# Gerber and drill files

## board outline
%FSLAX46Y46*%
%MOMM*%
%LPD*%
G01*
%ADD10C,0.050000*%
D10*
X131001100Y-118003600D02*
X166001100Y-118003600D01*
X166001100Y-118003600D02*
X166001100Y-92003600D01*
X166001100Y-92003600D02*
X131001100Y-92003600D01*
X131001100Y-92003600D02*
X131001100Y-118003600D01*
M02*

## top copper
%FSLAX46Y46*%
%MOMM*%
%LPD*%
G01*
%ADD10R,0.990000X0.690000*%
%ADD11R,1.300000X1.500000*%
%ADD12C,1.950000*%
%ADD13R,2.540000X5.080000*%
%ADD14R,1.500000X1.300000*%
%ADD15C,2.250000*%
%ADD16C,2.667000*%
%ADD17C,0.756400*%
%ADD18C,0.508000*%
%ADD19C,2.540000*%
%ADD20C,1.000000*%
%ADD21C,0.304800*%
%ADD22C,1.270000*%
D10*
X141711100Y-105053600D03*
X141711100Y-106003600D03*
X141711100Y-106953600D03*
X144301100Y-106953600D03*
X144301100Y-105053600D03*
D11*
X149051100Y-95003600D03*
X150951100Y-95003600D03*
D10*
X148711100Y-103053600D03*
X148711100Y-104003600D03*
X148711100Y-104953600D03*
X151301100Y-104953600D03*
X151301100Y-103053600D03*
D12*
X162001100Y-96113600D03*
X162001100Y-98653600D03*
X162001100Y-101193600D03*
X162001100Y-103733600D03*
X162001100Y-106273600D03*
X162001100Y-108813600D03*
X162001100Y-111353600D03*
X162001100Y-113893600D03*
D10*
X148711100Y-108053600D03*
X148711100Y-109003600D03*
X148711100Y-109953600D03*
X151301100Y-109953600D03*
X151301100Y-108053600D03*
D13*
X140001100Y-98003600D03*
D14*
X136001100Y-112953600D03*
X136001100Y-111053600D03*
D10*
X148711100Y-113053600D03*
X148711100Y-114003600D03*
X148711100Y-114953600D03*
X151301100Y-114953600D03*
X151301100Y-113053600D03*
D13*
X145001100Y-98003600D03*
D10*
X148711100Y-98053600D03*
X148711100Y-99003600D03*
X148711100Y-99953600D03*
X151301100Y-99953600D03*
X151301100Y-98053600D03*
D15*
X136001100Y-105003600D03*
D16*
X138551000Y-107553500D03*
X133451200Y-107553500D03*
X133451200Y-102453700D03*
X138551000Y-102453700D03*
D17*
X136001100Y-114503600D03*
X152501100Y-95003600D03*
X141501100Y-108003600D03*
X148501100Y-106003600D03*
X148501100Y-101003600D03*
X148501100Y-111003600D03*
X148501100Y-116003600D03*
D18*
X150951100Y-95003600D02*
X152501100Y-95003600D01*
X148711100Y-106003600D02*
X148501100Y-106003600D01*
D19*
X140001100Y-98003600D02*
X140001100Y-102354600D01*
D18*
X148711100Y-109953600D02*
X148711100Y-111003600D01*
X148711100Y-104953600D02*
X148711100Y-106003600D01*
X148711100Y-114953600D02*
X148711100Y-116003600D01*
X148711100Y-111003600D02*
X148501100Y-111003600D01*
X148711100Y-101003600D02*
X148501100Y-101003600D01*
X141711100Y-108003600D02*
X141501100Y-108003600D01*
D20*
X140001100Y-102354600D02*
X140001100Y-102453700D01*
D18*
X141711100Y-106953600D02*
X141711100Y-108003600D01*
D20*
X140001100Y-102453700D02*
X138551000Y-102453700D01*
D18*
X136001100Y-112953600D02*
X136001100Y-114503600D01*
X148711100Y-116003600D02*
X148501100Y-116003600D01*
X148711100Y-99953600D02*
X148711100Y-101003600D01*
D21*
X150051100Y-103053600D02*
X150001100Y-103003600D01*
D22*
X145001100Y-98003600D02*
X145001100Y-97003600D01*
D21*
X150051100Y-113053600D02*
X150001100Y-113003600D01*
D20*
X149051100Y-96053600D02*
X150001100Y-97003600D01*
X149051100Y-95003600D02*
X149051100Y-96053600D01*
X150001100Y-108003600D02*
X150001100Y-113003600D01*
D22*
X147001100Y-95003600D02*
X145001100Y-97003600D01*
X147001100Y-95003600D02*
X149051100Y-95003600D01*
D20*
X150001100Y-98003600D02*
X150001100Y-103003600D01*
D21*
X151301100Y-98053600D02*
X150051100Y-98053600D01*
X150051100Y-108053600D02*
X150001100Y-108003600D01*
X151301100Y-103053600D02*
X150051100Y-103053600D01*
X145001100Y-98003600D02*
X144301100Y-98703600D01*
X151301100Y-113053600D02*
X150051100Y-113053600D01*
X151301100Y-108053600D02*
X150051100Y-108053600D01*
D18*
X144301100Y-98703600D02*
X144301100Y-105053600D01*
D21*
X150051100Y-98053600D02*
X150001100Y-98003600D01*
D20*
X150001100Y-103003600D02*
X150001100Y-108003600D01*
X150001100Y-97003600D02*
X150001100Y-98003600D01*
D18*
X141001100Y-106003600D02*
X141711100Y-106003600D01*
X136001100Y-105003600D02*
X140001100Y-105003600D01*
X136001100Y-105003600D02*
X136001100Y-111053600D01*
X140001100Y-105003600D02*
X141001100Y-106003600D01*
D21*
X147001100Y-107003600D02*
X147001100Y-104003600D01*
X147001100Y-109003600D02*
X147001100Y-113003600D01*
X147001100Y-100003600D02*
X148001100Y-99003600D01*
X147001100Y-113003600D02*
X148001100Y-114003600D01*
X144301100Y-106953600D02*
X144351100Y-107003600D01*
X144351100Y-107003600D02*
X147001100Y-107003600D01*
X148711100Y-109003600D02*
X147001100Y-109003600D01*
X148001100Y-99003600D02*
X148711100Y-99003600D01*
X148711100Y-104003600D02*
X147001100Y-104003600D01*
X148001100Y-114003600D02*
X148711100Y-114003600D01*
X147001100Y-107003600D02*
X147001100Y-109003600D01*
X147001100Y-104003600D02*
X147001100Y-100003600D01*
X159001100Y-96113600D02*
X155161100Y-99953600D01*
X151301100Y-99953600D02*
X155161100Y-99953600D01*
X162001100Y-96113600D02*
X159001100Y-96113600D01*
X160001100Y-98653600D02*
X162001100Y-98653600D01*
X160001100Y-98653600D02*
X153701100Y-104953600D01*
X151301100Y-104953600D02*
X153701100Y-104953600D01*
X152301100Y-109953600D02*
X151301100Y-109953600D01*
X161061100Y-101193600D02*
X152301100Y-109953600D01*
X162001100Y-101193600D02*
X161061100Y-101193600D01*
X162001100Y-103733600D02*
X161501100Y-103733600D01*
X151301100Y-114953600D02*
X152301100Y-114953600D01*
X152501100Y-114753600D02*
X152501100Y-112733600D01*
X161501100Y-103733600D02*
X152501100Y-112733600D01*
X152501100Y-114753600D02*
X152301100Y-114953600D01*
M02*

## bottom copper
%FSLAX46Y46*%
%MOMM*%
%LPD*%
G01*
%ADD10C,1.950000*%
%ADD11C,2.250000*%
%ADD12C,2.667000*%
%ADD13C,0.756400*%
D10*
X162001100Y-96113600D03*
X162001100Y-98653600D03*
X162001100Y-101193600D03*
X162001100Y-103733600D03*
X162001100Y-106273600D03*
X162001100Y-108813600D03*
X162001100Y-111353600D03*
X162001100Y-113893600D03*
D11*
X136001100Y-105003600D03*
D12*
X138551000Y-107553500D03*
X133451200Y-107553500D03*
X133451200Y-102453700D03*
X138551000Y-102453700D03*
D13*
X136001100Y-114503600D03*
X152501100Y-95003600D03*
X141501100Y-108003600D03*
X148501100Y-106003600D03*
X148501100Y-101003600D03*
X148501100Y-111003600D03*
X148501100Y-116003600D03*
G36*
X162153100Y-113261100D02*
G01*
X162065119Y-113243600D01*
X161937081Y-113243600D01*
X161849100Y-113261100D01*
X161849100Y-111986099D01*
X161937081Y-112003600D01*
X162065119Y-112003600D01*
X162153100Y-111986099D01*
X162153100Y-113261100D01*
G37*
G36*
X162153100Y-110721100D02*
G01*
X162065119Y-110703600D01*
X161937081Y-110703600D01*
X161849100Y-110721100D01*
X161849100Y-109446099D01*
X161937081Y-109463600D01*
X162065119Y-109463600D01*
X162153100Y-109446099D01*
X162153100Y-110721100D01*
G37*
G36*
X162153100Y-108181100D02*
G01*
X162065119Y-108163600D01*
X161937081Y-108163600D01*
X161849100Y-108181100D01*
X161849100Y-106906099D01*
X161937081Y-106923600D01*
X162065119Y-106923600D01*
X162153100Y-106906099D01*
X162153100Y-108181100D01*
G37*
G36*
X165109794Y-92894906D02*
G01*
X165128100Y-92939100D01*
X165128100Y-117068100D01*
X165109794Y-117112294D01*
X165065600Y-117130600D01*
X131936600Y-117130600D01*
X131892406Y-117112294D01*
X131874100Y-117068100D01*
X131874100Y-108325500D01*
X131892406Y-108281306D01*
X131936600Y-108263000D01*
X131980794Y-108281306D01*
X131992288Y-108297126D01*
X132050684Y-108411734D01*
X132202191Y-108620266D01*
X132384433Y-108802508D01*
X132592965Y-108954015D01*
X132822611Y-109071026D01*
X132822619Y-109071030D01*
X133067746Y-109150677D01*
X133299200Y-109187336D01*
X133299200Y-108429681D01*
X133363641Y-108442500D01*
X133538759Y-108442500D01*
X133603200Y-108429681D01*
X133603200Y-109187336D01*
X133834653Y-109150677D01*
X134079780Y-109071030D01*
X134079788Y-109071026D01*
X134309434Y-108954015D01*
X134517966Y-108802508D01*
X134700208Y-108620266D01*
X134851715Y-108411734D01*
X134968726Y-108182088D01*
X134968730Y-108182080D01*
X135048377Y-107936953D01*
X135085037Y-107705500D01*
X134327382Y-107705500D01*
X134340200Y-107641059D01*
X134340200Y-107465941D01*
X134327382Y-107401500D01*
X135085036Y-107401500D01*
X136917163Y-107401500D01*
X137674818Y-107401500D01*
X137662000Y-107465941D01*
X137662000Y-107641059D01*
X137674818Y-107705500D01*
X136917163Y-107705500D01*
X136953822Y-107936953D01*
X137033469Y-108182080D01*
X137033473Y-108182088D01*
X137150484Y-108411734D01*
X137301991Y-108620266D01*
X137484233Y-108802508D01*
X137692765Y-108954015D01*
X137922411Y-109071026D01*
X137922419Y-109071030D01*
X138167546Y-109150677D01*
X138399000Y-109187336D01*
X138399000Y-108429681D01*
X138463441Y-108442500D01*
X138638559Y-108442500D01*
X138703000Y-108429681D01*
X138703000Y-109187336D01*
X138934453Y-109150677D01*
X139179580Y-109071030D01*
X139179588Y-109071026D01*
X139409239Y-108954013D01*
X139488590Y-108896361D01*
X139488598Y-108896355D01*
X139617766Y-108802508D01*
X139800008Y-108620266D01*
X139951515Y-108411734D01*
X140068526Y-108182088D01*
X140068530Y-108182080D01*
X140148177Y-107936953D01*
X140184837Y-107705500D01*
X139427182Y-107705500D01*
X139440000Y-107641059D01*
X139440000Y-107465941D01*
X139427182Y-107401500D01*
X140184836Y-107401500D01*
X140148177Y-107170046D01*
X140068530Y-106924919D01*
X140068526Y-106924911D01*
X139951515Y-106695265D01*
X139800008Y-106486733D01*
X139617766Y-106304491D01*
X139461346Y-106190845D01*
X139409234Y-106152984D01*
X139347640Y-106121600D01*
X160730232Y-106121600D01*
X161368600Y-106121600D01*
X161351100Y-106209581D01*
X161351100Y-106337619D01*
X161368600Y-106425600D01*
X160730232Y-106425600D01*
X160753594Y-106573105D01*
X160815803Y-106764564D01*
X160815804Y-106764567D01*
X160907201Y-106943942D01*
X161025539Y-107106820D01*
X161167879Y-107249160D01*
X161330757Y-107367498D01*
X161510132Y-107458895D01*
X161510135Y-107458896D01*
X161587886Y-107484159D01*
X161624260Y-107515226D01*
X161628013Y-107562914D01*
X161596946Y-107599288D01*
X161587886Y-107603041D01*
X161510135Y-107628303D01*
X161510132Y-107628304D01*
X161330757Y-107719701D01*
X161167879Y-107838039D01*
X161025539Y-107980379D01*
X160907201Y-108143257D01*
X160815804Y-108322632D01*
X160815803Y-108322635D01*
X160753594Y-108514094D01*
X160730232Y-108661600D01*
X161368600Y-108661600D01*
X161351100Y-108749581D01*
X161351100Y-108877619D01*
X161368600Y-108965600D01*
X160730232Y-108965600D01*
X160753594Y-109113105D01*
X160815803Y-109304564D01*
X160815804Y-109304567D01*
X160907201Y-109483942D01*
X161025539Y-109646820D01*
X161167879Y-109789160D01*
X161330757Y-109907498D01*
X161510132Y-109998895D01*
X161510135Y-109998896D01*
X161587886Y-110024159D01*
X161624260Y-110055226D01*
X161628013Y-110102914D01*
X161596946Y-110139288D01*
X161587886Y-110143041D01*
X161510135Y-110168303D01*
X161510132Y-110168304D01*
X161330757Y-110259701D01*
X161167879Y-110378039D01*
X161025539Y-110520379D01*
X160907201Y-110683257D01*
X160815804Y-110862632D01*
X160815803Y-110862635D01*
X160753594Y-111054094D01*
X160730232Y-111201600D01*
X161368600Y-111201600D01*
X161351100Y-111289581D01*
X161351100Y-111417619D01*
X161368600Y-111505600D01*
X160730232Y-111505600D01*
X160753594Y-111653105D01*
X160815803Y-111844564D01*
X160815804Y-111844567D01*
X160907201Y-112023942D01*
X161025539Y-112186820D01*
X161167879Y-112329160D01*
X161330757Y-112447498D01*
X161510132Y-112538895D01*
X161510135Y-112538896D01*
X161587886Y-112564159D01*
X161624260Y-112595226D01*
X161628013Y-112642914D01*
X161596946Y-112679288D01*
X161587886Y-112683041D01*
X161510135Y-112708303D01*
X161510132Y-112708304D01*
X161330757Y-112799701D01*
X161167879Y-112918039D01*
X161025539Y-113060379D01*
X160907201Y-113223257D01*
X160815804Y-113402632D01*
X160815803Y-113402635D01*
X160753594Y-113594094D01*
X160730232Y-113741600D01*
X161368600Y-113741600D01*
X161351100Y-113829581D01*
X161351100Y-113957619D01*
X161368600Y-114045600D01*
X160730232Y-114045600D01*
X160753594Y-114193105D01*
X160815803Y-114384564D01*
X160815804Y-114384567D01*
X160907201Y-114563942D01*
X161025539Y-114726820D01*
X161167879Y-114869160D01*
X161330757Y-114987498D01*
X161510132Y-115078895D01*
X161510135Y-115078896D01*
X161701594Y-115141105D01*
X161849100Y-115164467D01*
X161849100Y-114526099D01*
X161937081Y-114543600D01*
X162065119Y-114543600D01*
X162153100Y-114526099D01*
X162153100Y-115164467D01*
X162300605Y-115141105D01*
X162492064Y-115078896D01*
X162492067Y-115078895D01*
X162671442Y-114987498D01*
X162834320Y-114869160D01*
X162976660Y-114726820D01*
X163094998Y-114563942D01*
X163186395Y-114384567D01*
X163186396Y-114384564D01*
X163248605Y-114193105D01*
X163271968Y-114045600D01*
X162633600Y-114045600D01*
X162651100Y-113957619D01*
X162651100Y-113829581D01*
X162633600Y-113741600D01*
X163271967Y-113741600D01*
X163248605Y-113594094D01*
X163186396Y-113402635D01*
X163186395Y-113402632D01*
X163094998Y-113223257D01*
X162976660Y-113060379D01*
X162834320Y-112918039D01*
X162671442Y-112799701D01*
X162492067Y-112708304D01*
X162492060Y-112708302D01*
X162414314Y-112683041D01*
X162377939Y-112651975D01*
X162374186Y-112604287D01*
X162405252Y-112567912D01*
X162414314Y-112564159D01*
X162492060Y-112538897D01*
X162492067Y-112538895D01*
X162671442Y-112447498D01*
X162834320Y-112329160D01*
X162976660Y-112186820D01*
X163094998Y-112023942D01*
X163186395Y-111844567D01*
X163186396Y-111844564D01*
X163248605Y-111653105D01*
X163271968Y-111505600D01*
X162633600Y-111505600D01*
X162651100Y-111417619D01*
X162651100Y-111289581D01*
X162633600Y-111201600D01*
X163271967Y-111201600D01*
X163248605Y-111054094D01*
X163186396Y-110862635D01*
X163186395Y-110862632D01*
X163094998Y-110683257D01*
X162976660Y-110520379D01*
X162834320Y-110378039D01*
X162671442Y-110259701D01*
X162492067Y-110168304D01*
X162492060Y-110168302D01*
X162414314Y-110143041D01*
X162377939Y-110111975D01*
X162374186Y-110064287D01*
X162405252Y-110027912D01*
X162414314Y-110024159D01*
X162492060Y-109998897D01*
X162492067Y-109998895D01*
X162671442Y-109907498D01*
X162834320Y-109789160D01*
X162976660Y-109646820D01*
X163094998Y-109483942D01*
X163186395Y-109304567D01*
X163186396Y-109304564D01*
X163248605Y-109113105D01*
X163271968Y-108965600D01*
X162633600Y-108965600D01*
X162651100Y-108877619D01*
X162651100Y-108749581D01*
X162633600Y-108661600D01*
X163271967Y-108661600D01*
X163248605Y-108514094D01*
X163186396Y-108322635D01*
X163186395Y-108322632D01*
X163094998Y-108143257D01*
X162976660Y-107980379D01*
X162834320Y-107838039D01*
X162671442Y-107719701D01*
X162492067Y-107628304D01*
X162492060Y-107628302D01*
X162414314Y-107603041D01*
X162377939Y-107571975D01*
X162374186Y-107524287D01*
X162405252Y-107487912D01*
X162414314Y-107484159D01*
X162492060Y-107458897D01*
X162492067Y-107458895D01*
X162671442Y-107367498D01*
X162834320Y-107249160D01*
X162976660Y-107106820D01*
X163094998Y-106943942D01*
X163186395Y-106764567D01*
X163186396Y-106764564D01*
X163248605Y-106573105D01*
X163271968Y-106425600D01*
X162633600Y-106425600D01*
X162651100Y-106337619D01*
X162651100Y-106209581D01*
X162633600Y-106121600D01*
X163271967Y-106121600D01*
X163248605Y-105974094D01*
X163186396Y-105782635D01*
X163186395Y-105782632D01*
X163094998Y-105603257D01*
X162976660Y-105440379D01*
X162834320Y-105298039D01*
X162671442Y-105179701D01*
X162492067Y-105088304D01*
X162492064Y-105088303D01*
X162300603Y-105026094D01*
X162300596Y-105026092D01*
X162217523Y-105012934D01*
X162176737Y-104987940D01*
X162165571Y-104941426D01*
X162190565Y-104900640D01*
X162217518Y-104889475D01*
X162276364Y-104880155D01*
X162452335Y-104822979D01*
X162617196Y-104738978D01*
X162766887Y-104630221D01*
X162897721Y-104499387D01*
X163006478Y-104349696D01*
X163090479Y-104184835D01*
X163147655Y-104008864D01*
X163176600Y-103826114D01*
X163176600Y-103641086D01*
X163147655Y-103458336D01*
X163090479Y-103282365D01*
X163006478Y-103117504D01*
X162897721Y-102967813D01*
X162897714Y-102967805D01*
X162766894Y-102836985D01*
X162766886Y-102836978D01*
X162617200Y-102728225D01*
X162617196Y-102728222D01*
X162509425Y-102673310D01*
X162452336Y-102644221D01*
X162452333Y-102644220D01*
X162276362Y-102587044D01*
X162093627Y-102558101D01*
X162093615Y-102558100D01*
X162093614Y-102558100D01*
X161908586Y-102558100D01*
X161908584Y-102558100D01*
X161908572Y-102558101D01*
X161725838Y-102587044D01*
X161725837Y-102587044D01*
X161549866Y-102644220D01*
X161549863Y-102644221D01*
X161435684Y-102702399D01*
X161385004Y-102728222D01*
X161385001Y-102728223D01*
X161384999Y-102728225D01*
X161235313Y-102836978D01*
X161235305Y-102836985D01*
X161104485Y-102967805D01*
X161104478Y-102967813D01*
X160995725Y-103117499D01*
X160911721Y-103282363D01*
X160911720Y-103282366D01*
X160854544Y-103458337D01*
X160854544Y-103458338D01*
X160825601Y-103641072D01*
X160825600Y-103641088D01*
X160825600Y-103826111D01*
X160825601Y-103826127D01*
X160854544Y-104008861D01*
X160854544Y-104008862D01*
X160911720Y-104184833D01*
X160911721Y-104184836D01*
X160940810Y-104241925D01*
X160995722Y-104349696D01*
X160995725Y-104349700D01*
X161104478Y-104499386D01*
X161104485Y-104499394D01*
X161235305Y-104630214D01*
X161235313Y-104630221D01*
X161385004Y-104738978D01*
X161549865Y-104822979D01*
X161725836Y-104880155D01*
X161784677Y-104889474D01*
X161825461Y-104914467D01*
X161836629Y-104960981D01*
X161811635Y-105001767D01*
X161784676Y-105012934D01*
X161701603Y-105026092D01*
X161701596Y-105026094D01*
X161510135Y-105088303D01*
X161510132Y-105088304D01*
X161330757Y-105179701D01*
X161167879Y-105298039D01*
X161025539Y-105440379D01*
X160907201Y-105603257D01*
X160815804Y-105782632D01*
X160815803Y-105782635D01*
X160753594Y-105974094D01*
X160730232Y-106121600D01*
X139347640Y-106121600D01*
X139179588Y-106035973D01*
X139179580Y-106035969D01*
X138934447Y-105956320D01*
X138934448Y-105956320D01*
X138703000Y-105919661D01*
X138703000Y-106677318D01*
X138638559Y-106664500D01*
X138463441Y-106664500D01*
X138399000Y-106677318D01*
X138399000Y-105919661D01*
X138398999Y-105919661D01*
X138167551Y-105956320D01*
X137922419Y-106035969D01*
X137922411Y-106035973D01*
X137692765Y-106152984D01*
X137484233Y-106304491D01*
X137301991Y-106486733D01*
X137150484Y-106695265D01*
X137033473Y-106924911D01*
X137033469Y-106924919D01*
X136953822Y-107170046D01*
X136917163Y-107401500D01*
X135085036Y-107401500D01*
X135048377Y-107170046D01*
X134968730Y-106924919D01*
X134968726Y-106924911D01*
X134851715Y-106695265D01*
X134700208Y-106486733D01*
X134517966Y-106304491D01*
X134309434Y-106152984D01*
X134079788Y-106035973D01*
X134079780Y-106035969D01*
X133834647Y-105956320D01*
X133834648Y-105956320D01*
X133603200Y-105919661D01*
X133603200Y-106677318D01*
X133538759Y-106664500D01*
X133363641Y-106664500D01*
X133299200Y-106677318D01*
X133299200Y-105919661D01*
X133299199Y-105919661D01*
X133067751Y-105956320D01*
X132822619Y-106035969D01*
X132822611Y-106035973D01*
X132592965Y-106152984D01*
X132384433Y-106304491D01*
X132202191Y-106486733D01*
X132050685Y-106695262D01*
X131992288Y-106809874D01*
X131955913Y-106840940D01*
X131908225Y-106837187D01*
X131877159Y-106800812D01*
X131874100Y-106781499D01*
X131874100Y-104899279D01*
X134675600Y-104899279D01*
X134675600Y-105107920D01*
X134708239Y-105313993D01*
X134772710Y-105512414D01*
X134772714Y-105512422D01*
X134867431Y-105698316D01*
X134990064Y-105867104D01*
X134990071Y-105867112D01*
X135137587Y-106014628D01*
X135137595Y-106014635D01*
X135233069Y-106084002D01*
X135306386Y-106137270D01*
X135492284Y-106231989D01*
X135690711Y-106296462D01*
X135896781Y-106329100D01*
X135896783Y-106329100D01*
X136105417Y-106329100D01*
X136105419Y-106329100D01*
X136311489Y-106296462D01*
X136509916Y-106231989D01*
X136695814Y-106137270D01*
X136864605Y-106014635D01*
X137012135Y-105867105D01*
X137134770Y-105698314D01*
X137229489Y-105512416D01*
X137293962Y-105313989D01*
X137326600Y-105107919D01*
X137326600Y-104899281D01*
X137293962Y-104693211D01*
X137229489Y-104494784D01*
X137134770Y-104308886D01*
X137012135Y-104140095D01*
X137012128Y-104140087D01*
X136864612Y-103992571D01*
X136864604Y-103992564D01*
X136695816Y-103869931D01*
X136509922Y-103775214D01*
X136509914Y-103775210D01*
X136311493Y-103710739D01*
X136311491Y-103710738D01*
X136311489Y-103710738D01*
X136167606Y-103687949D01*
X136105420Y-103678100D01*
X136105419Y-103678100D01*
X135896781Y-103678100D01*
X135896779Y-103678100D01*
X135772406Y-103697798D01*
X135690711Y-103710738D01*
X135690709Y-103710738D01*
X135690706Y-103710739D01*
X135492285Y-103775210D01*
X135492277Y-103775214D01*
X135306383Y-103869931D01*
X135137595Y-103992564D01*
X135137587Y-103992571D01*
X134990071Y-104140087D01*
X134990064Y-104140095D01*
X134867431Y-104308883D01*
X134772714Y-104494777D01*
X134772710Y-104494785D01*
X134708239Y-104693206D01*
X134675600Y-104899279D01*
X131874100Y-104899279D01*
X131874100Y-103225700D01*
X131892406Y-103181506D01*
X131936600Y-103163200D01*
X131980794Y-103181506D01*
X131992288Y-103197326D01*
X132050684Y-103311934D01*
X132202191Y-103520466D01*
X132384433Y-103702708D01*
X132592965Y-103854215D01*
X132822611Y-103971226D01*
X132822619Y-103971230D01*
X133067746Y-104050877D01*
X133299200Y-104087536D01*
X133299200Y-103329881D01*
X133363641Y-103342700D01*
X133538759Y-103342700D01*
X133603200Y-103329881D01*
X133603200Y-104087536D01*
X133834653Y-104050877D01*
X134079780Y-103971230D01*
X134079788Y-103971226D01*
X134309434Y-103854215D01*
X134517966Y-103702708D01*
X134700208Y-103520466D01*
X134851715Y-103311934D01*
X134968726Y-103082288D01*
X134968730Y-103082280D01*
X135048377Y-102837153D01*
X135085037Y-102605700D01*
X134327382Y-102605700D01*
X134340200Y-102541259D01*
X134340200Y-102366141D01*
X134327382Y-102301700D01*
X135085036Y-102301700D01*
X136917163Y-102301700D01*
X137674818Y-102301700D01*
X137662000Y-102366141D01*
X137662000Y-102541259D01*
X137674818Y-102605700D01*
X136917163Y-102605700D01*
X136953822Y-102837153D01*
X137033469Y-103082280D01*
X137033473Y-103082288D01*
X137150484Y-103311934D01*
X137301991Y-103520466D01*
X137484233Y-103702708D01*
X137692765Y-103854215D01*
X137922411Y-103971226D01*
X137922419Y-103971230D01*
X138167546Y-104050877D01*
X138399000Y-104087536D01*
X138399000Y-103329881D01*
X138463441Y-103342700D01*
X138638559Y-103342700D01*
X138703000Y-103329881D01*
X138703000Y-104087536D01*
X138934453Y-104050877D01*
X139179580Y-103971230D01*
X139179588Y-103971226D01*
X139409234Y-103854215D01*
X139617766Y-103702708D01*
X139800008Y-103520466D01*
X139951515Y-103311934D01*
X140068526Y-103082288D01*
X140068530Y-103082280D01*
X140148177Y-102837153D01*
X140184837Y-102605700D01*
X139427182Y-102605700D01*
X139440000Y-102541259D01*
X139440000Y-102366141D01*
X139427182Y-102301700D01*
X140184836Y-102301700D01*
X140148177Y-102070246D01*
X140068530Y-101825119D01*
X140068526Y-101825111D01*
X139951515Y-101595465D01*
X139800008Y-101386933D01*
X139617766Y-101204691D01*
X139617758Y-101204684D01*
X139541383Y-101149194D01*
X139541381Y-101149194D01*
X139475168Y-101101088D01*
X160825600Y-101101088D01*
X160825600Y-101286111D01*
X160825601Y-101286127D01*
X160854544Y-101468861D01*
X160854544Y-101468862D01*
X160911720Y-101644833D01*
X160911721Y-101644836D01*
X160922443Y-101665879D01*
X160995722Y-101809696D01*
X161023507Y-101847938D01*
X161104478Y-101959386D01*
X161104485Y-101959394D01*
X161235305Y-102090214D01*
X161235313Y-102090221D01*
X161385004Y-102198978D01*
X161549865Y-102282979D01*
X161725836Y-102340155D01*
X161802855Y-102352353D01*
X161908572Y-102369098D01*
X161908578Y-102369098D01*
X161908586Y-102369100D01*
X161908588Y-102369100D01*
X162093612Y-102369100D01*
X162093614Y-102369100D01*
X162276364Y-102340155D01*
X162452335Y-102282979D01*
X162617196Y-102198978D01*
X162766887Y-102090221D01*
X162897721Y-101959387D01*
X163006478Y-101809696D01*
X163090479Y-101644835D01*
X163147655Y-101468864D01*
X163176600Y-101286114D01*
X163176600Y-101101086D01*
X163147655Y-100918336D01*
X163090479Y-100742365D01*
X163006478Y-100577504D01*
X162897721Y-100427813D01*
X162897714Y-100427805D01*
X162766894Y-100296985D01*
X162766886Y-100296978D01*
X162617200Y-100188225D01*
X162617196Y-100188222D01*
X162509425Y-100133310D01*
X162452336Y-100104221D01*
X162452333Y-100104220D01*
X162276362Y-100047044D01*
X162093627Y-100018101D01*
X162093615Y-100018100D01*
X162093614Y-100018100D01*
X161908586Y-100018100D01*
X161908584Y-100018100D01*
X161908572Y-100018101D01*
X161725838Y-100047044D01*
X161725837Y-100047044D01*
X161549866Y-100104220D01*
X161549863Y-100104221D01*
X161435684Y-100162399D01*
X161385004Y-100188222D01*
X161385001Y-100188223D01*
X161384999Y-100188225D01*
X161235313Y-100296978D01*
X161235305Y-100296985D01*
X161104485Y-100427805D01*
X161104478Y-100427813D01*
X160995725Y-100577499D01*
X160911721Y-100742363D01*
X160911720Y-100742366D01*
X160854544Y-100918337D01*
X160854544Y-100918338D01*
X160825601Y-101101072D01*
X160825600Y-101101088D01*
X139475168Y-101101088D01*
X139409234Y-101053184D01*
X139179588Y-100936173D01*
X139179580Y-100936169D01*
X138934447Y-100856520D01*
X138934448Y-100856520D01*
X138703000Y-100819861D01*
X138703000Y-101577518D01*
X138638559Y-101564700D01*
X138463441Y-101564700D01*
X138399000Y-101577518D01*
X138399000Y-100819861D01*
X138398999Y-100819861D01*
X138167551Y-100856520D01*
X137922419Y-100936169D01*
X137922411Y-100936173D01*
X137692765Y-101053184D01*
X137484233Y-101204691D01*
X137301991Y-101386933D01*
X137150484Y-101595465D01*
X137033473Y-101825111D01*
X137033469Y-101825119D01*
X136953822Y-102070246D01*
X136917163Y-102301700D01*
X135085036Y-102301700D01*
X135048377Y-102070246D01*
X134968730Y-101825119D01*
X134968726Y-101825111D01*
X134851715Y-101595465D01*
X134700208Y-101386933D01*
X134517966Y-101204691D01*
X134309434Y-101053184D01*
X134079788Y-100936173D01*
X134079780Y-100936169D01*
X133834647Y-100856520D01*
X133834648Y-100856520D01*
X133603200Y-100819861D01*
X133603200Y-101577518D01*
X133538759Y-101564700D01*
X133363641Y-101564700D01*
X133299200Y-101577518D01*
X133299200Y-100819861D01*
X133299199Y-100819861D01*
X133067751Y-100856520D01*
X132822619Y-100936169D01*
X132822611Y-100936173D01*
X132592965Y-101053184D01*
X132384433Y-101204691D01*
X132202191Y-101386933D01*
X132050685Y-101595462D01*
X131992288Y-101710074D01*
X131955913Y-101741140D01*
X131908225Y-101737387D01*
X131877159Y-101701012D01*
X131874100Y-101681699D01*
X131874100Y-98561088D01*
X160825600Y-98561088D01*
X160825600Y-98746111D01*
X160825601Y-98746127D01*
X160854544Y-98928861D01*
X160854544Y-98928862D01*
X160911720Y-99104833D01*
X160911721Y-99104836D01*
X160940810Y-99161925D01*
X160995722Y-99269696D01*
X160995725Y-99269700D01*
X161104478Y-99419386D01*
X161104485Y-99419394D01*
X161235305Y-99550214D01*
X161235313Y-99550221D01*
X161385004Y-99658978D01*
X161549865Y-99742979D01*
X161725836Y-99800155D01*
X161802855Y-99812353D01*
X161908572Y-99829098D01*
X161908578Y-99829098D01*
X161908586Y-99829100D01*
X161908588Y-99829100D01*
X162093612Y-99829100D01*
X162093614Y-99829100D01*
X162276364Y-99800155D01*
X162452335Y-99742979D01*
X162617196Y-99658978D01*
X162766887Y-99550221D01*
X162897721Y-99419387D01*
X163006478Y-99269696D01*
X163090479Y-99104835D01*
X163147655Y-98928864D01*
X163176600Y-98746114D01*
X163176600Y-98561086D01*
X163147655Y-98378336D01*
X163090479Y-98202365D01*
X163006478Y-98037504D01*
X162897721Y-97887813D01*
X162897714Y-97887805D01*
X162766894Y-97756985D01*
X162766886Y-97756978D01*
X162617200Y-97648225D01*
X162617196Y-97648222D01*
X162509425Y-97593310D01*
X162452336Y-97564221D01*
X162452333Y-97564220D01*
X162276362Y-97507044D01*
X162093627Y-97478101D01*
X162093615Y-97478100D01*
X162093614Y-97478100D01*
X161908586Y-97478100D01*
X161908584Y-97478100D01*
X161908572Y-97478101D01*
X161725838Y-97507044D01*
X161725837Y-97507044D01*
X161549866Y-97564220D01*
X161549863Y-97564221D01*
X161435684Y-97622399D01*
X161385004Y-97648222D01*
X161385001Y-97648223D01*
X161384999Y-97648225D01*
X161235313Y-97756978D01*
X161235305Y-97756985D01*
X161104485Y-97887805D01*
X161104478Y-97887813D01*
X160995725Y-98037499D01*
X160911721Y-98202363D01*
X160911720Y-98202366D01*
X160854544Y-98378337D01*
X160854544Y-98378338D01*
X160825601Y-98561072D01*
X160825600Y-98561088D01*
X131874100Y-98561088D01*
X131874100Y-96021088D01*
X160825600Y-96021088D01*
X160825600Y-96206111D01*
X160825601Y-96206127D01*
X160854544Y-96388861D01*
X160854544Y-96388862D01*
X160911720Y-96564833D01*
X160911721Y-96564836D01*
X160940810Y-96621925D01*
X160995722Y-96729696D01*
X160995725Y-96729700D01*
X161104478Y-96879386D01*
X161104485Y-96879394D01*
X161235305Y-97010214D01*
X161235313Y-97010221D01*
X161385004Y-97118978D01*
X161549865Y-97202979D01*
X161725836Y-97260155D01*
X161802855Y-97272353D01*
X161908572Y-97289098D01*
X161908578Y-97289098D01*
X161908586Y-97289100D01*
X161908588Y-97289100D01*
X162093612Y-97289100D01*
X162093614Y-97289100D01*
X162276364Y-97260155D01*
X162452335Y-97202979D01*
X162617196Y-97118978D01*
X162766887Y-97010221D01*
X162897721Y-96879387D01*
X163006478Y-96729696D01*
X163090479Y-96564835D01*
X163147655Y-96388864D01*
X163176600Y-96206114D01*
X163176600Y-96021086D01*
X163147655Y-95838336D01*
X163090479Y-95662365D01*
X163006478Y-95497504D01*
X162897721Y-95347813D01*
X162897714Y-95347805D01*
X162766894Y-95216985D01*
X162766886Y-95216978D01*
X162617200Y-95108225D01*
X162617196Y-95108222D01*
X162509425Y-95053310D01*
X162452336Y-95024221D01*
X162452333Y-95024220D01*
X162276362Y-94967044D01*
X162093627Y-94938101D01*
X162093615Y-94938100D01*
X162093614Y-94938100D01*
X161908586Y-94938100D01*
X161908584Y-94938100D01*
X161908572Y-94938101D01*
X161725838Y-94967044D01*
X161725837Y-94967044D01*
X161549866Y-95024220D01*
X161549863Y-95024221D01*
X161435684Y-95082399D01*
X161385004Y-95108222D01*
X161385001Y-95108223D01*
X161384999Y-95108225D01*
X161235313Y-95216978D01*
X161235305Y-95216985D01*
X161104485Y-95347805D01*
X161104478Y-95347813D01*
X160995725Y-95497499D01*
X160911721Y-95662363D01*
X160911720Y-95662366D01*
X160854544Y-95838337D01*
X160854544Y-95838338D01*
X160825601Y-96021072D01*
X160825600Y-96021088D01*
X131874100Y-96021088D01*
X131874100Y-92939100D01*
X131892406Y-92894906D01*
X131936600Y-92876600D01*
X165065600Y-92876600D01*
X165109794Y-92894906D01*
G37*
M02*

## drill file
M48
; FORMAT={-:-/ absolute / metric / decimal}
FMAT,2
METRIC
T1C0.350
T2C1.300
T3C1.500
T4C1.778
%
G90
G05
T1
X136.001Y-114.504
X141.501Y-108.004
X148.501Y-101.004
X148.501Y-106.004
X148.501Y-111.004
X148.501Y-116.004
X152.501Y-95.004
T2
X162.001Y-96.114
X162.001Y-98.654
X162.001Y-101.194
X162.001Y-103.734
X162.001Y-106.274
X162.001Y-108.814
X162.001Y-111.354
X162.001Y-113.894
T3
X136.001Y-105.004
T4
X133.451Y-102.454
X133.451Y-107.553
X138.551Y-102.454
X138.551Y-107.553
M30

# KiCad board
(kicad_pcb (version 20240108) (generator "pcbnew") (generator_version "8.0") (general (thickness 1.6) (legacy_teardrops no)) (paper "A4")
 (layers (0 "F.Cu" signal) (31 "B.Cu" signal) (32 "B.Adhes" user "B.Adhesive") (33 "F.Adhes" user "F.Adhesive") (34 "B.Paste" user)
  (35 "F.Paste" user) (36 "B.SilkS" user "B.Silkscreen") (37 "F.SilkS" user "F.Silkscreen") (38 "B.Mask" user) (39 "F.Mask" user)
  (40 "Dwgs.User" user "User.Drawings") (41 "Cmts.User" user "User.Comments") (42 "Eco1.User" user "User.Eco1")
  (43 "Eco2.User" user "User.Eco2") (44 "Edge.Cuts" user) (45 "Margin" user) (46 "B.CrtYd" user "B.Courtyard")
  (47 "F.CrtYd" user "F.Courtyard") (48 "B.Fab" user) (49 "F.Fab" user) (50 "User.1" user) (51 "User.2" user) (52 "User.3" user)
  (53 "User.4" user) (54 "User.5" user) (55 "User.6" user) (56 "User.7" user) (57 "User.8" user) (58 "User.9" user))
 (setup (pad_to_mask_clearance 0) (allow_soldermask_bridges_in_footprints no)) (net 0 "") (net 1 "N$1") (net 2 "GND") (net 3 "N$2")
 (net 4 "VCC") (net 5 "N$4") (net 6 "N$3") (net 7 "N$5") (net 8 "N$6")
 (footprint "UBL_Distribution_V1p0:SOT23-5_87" (layer "F.Cu") (at 143.0011 106.0036 -90)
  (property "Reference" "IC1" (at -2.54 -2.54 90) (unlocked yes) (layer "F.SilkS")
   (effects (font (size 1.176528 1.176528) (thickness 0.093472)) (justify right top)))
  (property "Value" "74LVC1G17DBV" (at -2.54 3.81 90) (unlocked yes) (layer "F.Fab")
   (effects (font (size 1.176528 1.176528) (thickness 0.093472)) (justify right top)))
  (pad "1" smd rect (at -0.95 1.29 270) (size 0.69 0.99) (layers "F.Cu" "F.Paste" "F.Mask") (solder_mask_margin 0.1016)
   (thermal_bridge_angle 0))
  (pad "2" smd rect (at 0 1.29 270) (size 0.69 0.99) (layers "F.Cu" "F.Paste" "F.Mask") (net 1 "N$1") (solder_mask_margin 0.1016)
   (thermal_bridge_angle 0))
  (pad "3" smd rect (at 0.95 1.29 270) (size 0.69 0.99) (layers "F.Cu" "F.Paste" "F.Mask") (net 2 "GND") (solder_mask_margin 0.1016)
   (thermal_bridge_angle 0))
  (pad "4" smd rect (at 0.95 -1.3 270) (size 0.69 0.99) (layers "F.Cu" "F.Paste" "F.Mask") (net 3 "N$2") (solder_mask_margin 0.1016)
   (thermal_bridge_angle 0))
  (pad "5" smd rect (at -0.95 -1.3 270) (size 0.69 0.99) (layers "F.Cu" "F.Paste" "F.Mask") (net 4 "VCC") (solder_mask_margin 0.1016)
   (thermal_bridge_angle 0)))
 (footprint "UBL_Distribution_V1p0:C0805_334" (layer "F.Cu") (at 150.0011 95.0036)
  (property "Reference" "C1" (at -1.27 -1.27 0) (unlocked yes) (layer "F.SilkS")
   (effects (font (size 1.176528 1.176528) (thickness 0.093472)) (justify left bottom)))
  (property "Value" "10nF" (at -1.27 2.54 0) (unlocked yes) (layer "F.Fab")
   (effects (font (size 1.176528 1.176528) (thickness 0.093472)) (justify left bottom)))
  (pad "1" smd rect (at -0.95 0) (size 1.3 1.5) (layers "F.Cu" "F.Paste" "F.Mask") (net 4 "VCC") (solder_mask_margin 0.1016)
   (thermal_bridge_angle 0))
  (pad "2" smd rect (at 0.95 0) (size 1.3 1.5) (layers "F.Cu" "F.Paste" "F.Mask") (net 2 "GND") (solder_mask_margin 0.1016)
   (thermal_bridge_angle 0)))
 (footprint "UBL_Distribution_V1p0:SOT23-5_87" (layer "F.Cu") (at 150.0011 104.0036 -90)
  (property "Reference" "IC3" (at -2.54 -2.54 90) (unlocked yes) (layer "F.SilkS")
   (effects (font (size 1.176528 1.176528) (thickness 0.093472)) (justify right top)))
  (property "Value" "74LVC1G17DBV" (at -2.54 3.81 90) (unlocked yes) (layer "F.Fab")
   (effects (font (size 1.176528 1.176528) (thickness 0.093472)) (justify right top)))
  (pad "1" smd rect (at -0.95 1.29 270) (size 0.69 0.99) (layers "F.Cu" "F.Paste" "F.Mask") (solder_mask_margin 0.1016)
   (thermal_bridge_angle 0))
  (pad "2" smd rect (at 0 1.29 270) (size 0.69 0.99) (layers "F.Cu" "F.Paste" "F.Mask") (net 3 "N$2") (solder_mask_margin 0.1016)
   (thermal_bridge_angle 0))
  (pad "3" smd rect (at 0.95 1.29 270) (size 0.69 0.99) (layers "F.Cu" "F.Paste" "F.Mask") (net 2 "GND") (solder_mask_margin 0.1016)
   (thermal_bridge_angle 0))
  (pad "4" smd rect (at 0.95 -1.3 270) (size 0.69 0.99) (layers "F.Cu" "F.Paste" "F.Mask") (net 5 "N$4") (solder_mask_margin 0.1016)
   (thermal_bridge_angle 0))
  (pad "5" smd rect (at -0.95 -1.3 270) (size 0.69 0.99) (layers "F.Cu" "F.Paste" "F.Mask") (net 4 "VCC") (solder_mask_margin 0.1016)
   (thermal_bridge_angle 0)))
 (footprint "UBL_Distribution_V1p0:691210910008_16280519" (layer "F.Cu") (at 162.0011 105.0036 -90)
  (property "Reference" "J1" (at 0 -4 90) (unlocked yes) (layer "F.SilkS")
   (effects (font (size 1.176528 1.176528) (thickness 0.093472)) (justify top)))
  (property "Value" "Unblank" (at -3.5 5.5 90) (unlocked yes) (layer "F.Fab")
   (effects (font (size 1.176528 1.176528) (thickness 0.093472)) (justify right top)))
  (pad "1" thru_hole circle (at -8.89 0 270) (size 1.95 1.95) (drill 1.3) (layers "*.Cu" "*.Mask") (remove_unused_layers no) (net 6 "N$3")
   (solder_mask_margin 0.1016) (thermal_bridge_angle 0))
  (pad "2" thru_hole circle (at -6.35 0 270) (size 1.95 1.95) (drill 1.3) (layers "*.Cu" "*.Mask") (remove_unused_layers no) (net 5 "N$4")
   (solder_mask_margin 0.1016) (thermal_bridge_angle 0))
  (pad "3" thru_hole circle (at -3.81 0 270) (size 1.95 1.95) (drill 1.3) (layers "*.Cu" "*.Mask") (remove_unused_layers no) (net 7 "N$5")
   (solder_mask_margin 0.1016) (thermal_bridge_angle 0))
  (pad "4" thru_hole circle (at -1.27 0 270) (size 1.95 1.95) (drill 1.3) (layers "*.Cu" "*.Mask") (remove_unused_layers no) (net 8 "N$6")
   (solder_mask_margin 0.1016) (thermal_bridge_angle 0))
  (pad "5" thru_hole circle (at 1.27 0 270) (size 1.95 1.95) (drill 1.3) (layers "*.Cu" "*.Mask") (remove_unused_layers no) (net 2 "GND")
   (solder_mask_margin 0.1016) (thermal_bridge_angle 0))
  (pad "6" thru_hole circle (at 3.81 0 270) (size 1.95 1.95) (drill 1.3) (layers "*.Cu" "*.Mask") (remove_unused_layers no) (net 2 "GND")
   (solder_mask_margin 0.1016) (thermal_bridge_angle 0))
  (pad "7" thru_hole circle (at 6.35 0 270) (size 1.95 1.95) (drill 1.3) (layers "*.Cu" "*.Mask") (remove_unused_layers no) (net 2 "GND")
   (solder_mask_margin 0.1016) (thermal_bridge_angle 0))
  (pad "8" thru_hole circle (at 8.89 0 270) (size 1.95 1.95) (drill 1.3) (layers "*.Cu" "*.Mask") (remove_unused_layers no) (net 2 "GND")
   (solder_mask_margin 0.1016) (thermal_bridge_angle 0)))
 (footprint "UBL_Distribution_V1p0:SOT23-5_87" (layer "F.Cu") (at 150.0011 109.0036 -90)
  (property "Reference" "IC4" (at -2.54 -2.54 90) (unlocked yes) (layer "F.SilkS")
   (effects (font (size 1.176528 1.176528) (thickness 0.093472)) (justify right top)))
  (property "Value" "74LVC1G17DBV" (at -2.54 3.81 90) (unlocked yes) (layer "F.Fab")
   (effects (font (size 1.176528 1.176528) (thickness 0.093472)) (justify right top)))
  (pad "1" smd rect (at -0.95 1.29 270) (size 0.69 0.99) (layers "F.Cu" "F.Paste" "F.Mask") (solder_mask_margin 0.1016)
   (thermal_bridge_angle 0))
  (pad "2" smd rect (at 0 1.29 270) (size 0.69 0.99) (layers "F.Cu" "F.Paste" "F.Mask") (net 3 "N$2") (solder_mask_margin 0.1016)
   (thermal_bridge_angle 0))
  (pad "3" smd rect (at 0.95 1.29 270) (size 0.69 0.99) (layers "F.Cu" "F.Paste" "F.Mask") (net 2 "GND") (solder_mask_margin 0.1016)
   (thermal_bridge_angle 0))
  (pad "4" smd rect (at 0.95 -1.3 270) (size 0.69 0.99) (layers "F.Cu" "F.Paste" "F.Mask") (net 7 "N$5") (solder_mask_margin 0.1016)
   (thermal_bridge_angle 0))
  (pad "5" smd rect (at -0.95 -1.3 270) (size 0.69 0.99) (layers "F.Cu" "F.Paste" "F.Mask") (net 4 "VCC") (solder_mask_margin 0.1016)
   (thermal_bridge_angle 0)))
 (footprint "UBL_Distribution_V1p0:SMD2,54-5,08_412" (layer "F.Cu") (at 140.0011 98.0036)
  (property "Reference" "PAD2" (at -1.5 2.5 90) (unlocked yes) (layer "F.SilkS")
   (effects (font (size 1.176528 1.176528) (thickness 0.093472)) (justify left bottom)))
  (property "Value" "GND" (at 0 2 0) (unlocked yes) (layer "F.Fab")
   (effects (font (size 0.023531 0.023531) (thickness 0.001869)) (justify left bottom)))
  (pad "1" smd rect (at 0 0) (size 2.54 5.08) (layers "F.Cu" "F.Paste" "F.Mask") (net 2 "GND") (solder_mask_margin 0.1016)
   (thermal_bridge_angle 0)))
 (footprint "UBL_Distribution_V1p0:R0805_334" (layer "F.Cu") (at 136.0011 112.0036 90)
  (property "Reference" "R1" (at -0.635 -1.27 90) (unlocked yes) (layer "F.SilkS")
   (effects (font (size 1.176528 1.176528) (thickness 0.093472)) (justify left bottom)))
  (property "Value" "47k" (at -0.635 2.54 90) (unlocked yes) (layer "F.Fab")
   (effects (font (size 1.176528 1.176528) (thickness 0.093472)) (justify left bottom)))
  (pad "1" smd rect (at -0.95 0 90) (size 1.3 1.5) (layers "F.Cu" "F.Paste" "F.Mask") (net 2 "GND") (solder_mask_margin 0.1016)
   (thermal_bridge_angle 0))
  (pad "2" smd rect (at 0.95 0 90) (size 1.3 1.5) (layers "F.Cu" "F.Paste" "F.Mask") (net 1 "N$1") (solder_mask_margin 0.1016)
   (thermal_bridge_angle 0)))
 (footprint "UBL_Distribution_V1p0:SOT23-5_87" (layer "F.Cu") (at 150.0011 114.0036 -90)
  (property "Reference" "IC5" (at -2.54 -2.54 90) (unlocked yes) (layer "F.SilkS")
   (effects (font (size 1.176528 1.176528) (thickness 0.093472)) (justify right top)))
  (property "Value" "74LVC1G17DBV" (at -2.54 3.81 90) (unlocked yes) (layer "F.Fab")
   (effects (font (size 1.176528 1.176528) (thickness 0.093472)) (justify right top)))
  (pad "1" smd rect (at -0.95 1.29 270) (size 0.69 0.99) (layers "F.Cu" "F.Paste" "F.Mask") (solder_mask_margin 0.1016)
   (thermal_bridge_angle 0))
  (pad "2" smd rect (at 0 1.29 270) (size 0.69 0.99) (layers "F.Cu" "F.Paste" "F.Mask") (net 3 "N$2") (solder_mask_margin 0.1016)
   (thermal_bridge_angle 0))
  (pad "3" smd rect (at 0.95 1.29 270) (size 0.69 0.99) (layers "F.Cu" "F.Paste" "F.Mask") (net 2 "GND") (solder_mask_margin 0.1016)
   (thermal_bridge_angle 0))
  (pad "4" smd rect (at 0.95 -1.3 270) (size 0.69 0.99) (layers "F.Cu" "F.Paste" "F.Mask") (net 8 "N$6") (solder_mask_margin 0.1016)
   (thermal_bridge_angle 0))
  (pad "5" smd rect (at -0.95 -1.3 270) (size 0.69 0.99) (layers "F.Cu" "F.Paste" "F.Mask") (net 4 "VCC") (solder_mask_margin 0.1016)
   (thermal_bridge_angle 0)))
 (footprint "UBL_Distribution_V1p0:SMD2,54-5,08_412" (layer "F.Cu") (at 145.0011 98.0036)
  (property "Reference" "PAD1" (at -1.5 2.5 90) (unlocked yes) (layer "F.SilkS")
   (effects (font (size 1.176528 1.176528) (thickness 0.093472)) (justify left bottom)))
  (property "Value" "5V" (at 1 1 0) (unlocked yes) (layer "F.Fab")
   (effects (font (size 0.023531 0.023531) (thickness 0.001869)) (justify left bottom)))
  (pad "1" smd rect (at 0 0) (size 2.54 5.08) (layers "F.Cu" "F.Paste" "F.Mask") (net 4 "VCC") (solder_mask_margin 0.1016)
   (thermal_bridge_angle 0)))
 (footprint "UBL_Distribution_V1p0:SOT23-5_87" (layer "F.Cu") (at 150.0011 99.0036 -90)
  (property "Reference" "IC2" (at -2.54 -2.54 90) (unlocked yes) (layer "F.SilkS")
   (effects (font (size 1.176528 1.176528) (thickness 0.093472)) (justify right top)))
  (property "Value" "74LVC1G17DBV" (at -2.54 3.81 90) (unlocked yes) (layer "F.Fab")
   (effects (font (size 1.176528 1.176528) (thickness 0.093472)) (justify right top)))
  (pad "1" smd rect (at -0.95 1.29 270) (size 0.69 0.99) (layers "F.Cu" "F.Paste" "F.Mask") (solder_mask_margin 0.1016)
   (thermal_bridge_angle 0))
  (pad "2" smd rect (at 0 1.29 270) (size 0.69 0.99) (layers "F.Cu" "F.Paste" "F.Mask") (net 3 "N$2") (solder_mask_margin 0.1016)
   (thermal_bridge_angle 0))
  (pad "3" smd rect (at 0.95 1.29 270) (size 0.69 0.99) (layers "F.Cu" "F.Paste" "F.Mask") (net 2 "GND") (solder_mask_margin 0.1016)
   (thermal_bridge_angle 0))
  (pad "4" smd rect (at 0.95 -1.3 270) (size 0.69 0.99) (layers "F.Cu" "F.Paste" "F.Mask") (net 6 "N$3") (solder_mask_margin 0.1016)
   (thermal_bridge_angle 0))
  (pad "5" smd rect (at -0.95 -1.3 270) (size 0.69 0.99) (layers "F.Cu" "F.Paste" "F.Mask") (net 4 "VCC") (solder_mask_margin 0.1016)
   (thermal_bridge_angle 0)))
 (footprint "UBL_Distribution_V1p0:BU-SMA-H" (layer "F.Cu") (at 136.0011 105.0036 180)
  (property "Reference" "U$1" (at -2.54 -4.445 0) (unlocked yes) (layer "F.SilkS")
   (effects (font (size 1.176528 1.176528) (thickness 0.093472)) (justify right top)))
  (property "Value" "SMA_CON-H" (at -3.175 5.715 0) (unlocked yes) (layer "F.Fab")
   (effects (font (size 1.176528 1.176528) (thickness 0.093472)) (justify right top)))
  (pad "1" thru_hole circle (at 0 0 180) (size 2.25 2.25) (drill 1.5) (layers "*.Cu" "*.Mask") (remove_unused_layers no) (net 1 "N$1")
   (solder_mask_margin 0.1016) (thermal_bridge_angle 0))
  (pad "2" thru_hole circle (at -2.5499 -2.5499 180) (size 2.667 2.667) (drill 1.778) (layers "*.Cu" "*.Mask") (remove_unused_layers no)
   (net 2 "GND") (solder_mask_margin 0.1016) (thermal_bridge_angle 0))
  (pad "3" thru_hole circle (at 2.5499 -2.5499 180) (size 2.667 2.667) (drill 1.778) (layers "*.Cu" "*.Mask") (remove_unused_layers no)
   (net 2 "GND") (solder_mask_margin 0.1016) (thermal_bridge_angle 0))
  (pad "4" thru_hole circle (at 2.5499 2.5499 180) (size 2.667 2.667) (drill 1.778) (layers "*.Cu" "*.Mask") (remove_unused_layers no)
   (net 2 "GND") (solder_mask_margin 0.1016) (thermal_bridge_angle 0))
  (pad "5" thru_hole circle (at -2.5499 2.5499 180) (size 2.667 2.667) (drill 1.778) (layers "*.Cu" "*.Mask") (remove_unused_layers no)
   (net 2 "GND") (solder_mask_margin 0.1016) (thermal_bridge_angle 0)))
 (gr_line (start 131.0011 118.0036) (end 166.0011 118.0036) (stroke (width 0.05) (type solid)) (layer "Edge.Cuts"))
 (gr_line (start 166.0011 118.0036) (end 166.0011 92.0036) (stroke (width 0.05) (type solid)) (layer "Edge.Cuts"))
 (gr_line (start 166.0011 92.0036) (end 131.0011 92.0036) (stroke (width 0.05) (type solid)) (layer "Edge.Cuts"))
 (gr_line (start 131.0011 92.0036) (end 131.0011 118.0036) (stroke (width 0.05) (type solid)) (layer "Edge.Cuts"))
 (segment (start 150.9511 95.0036) (end 152.5011 95.0036) (width 0.508) (layer "F.Cu") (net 2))
 (segment (start 148.7111 106.0036) (end 148.5011 106.0036) (width 0.508) (layer "F.Cu") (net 2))
 (segment (start 140.0011 98.0036) (end 140.0011 102.3546) (width 2.54) (layer "F.Cu") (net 2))
 (segment (start 148.7111 109.9536) (end 148.7111 111.0036) (width 0.508) (layer "F.Cu") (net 2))
 (segment (start 148.7111 104.9536) (end 148.7111 106.0036) (width 0.508) (layer "F.Cu") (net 2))
 (segment (start 148.7111 114.9536) (end 148.7111 116.0036) (width 0.508) (layer "F.Cu") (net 2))
 (segment (start 148.7111 111.0036) (end 148.5011 111.0036) (width 0.508) (layer "F.Cu") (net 2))
 (segment (start 148.7111 101.0036) (end 148.5011 101.0036) (width 0.508) (layer "F.Cu") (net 2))
 (segment (start 141.7111 108.0036) (end 141.5011 108.0036) (width 0.508) (layer "F.Cu") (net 2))
 (segment (start 140.0011 102.3546) (end 140.0011 102.4537) (width 1) (layer "F.Cu") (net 2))
 (segment (start 141.7111 106.9536) (end 141.7111 108.0036) (width 0.508) (layer "F.Cu") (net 2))
 (segment (start 140.0011 102.4537) (end 138.551 102.4537) (width 1) (layer "F.Cu") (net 2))
 (segment (start 136.0011 112.9536) (end 136.0011 114.5036) (width 0.508) (layer "F.Cu") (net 2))
 (segment (start 148.7111 116.0036) (end 148.5011 116.0036) (width 0.508) (layer "F.Cu") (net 2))
 (segment (start 148.7111 99.9536) (end 148.7111 101.0036) (width 0.508) (layer "F.Cu") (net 2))
 (via (at 136.0011 114.5036) (size 0.7564) (drill 0.35) (layers "F.Cu" "B.Cu") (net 2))
 (via (at 152.5011 95.0036) (size 0.7564) (drill 0.35) (layers "F.Cu" "B.Cu") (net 2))
 (via (at 141.5011 108.0036) (size 0.7564) (drill 0.35) (layers "F.Cu" "B.Cu") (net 2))
 (via (at 148.5011 106.0036) (size 0.7564) (drill 0.35) (layers "F.Cu" "B.Cu") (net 2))
 (via (at 148.5011 101.0036) (size 0.7564) (drill 0.35) (layers "F.Cu" "B.Cu") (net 2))
 (via (at 148.5011 111.0036) (size 0.7564) (drill 0.35) (layers "F.Cu" "B.Cu") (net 2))
 (via (at 148.5011 116.0036) (size 0.7564) (drill 0.35) (layers "F.Cu" "B.Cu") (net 2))
 (segment (start 150.0511 103.0536) (end 150.0011 103.0036) (width 0.3048) (layer "F.Cu") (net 4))
 (segment (start 145.0011 98.0036) (end 145.0011 97.0036) (width 1.27) (layer "F.Cu") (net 4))
 (segment (start 150.0511 113.0536) (end 150.0011 113.0036) (width 0.3048) (layer "F.Cu") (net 4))
 (segment (start 149.0511 96.0536) (end 150.0011 97.0036) (width 1) (layer "F.Cu") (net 4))
 (segment (start 149.0511 95.0036) (end 149.0511 96.0536) (width 1) (layer "F.Cu") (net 4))
 (segment (start 150.0011 108.0036) (end 150.0011 113.0036) (width 1) (layer "F.Cu") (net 4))
 (segment (start 147.0011 95.0036) (end 145.0011 97.0036) (width 1.27) (layer "F.Cu") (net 4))
 (segment (start 147.0011 95.0036) (end 149.0511 95.0036) (width 1.27) (layer "F.Cu") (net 4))
 (segment (start 150.0011 98.0036) (end 150.0011 103.0036) (width 1) (layer "F.Cu") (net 4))
 (segment (start 151.3011 98.0536) (end 150.0511 98.0536) (width 0.3048) (layer "F.Cu") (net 4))
 (segment (start 150.0511 108.0536) (end 150.0011 108.0036) (width 0.3048) (layer "F.Cu") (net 4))
 (segment (start 151.3011 103.0536) (end 150.0511 103.0536) (width 0.3048) (layer "F.Cu") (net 4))
 (segment (start 145.0011 98.0036) (end 144.3011 98.7036) (width 0.3048) (layer "F.Cu") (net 4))
 (segment (start 151.3011 113.0536) (end 150.0511 113.0536) (width 0.3048) (layer "F.Cu") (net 4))
 (segment (start 151.3011 108.0536) (end 150.0511 108.0536) (width 0.3048) (layer "F.Cu") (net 4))
 (segment (start 144.3011 98.7036) (end 144.3011 105.0536) (width 0.508) (layer "F.Cu") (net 4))
 (segment (start 150.0511 98.0536) (end 150.0011 98.0036) (width 0.3048) (layer "F.Cu") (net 4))
 (segment (start 150.0011 103.0036) (end 150.0011 108.0036) (width 1) (layer "F.Cu") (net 4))
 (segment (start 150.0011 97.0036) (end 150.0011 98.0036) (width 1) (layer "F.Cu") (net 4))
 (segment (start 141.0011 106.0036) (end 141.7111 106.0036) (width 0.508) (layer "F.Cu") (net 1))
 (segment (start 136.0011 105.0036) (end 140.0011 105.0036) (width 0.508) (layer "F.Cu") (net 1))
 (segment (start 136.0011 105.0036) (end 136.0011 111.0536) (width 0.508) (layer "F.Cu") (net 1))
 (segment (start 140.0011 105.0036) (end 141.0011 106.0036) (width 0.508) (layer "F.Cu") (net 1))
 (segment (start 147.0011 107.0036) (end 147.0011 104.0036) (width 0.3048) (layer "F.Cu") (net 3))
 (segment (start 147.0011 109.0036) (end 147.0011 113.0036) (width 0.3048) (layer "F.Cu") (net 3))
 (segment (start 147.0011 100.0036) (end 148.0011 99.0036) (width 0.3048) (layer "F.Cu") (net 3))
 (segment (start 147.0011 113.0036) (end 148.0011 114.0036) (width 0.3048) (layer "F.Cu") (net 3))
 (segment (start 144.3011 106.9536) (end 144.3511 107.0036) (width 0.3048) (layer "F.Cu") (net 3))
 (segment (start 144.3511 107.0036) (end 147.0011 107.0036) (width 0.3048) (layer "F.Cu") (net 3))
 (segment (start 148.7111 109.0036) (end 147.0011 109.0036) (width 0.3048) (layer "F.Cu") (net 3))
 (segment (start 148.0011 99.0036) (end 148.7111 99.0036) (width 0.3048) (layer "F.Cu") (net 3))
 (segment (start 148.7111 104.0036) (end 147.0011 104.0036) (width 0.3048) (layer "F.Cu") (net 3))
 (segment (start 148.0011 114.0036) (end 148.7111 114.0036) (width 0.3048) (layer "F.Cu") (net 3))
 (segment (start 147.0011 107.0036) (end 147.0011 109.0036) (width 0.3048) (layer "F.Cu") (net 3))
 (segment (start 147.0011 104.0036) (end 147.0011 100.0036) (width 0.3048) (layer "F.Cu") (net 3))
 (segment (start 159.0011 96.1136) (end 155.1611 99.9536) (width 0.3048) (layer "F.Cu") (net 6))
 (segment (start 151.3011 99.9536) (end 155.1611 99.9536) (width 0.3048) (layer "F.Cu") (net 6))
 (segment (start 162.0011 96.1136) (end 159.0011 96.1136) (width 0.3048) (layer "F.Cu") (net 6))
 (segment (start 160.0011 98.6536) (end 162.0011 98.6536) (width 0.3048) (layer "F.Cu") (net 5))
 (segment (start 160.0011 98.6536) (end 153.7011 104.9536) (width 0.3048) (layer "F.Cu") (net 5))
 (segment (start 151.3011 104.9536) (end 153.7011 104.9536) (width 0.3048) (layer "F.Cu") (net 5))
 (segment (start 152.3011 109.9536) (end 151.3011 109.9536) (width 0.3048) (layer "F.Cu") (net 7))
 (segment (start 161.0611 101.1936) (end 152.3011 109.9536) (width 0.3048) (layer "F.Cu") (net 7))
 (segment (start 162.0011 101.1936) (end 161.0611 101.1936) (width 0.3048) (layer "F.Cu") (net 7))
 (segment (start 162.0011 103.7336) (end 161.5011 103.7336) (width 0.3048) (layer "F.Cu") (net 8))
 (segment (start 151.3011 114.9536) (end 152.3011 114.9536) (width 0.3048) (layer "F.Cu") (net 8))
 (segment (start 152.5011 114.7536) (end 152.5011 112.7336) (width 0.3048) (layer "F.Cu") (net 8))
 (segment (start 161.5011 103.7336) (end 152.5011 112.7336) (width 0.3048) (layer "F.Cu") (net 8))
 (segment (start 152.5011 114.7536) (end 152.3011 114.9536) (width 0.3048) (layer "F.Cu") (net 8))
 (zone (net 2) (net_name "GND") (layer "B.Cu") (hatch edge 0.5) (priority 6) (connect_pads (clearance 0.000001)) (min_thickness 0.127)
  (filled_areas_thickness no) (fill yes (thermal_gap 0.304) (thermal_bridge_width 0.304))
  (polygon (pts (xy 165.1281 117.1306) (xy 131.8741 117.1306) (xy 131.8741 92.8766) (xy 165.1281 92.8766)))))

